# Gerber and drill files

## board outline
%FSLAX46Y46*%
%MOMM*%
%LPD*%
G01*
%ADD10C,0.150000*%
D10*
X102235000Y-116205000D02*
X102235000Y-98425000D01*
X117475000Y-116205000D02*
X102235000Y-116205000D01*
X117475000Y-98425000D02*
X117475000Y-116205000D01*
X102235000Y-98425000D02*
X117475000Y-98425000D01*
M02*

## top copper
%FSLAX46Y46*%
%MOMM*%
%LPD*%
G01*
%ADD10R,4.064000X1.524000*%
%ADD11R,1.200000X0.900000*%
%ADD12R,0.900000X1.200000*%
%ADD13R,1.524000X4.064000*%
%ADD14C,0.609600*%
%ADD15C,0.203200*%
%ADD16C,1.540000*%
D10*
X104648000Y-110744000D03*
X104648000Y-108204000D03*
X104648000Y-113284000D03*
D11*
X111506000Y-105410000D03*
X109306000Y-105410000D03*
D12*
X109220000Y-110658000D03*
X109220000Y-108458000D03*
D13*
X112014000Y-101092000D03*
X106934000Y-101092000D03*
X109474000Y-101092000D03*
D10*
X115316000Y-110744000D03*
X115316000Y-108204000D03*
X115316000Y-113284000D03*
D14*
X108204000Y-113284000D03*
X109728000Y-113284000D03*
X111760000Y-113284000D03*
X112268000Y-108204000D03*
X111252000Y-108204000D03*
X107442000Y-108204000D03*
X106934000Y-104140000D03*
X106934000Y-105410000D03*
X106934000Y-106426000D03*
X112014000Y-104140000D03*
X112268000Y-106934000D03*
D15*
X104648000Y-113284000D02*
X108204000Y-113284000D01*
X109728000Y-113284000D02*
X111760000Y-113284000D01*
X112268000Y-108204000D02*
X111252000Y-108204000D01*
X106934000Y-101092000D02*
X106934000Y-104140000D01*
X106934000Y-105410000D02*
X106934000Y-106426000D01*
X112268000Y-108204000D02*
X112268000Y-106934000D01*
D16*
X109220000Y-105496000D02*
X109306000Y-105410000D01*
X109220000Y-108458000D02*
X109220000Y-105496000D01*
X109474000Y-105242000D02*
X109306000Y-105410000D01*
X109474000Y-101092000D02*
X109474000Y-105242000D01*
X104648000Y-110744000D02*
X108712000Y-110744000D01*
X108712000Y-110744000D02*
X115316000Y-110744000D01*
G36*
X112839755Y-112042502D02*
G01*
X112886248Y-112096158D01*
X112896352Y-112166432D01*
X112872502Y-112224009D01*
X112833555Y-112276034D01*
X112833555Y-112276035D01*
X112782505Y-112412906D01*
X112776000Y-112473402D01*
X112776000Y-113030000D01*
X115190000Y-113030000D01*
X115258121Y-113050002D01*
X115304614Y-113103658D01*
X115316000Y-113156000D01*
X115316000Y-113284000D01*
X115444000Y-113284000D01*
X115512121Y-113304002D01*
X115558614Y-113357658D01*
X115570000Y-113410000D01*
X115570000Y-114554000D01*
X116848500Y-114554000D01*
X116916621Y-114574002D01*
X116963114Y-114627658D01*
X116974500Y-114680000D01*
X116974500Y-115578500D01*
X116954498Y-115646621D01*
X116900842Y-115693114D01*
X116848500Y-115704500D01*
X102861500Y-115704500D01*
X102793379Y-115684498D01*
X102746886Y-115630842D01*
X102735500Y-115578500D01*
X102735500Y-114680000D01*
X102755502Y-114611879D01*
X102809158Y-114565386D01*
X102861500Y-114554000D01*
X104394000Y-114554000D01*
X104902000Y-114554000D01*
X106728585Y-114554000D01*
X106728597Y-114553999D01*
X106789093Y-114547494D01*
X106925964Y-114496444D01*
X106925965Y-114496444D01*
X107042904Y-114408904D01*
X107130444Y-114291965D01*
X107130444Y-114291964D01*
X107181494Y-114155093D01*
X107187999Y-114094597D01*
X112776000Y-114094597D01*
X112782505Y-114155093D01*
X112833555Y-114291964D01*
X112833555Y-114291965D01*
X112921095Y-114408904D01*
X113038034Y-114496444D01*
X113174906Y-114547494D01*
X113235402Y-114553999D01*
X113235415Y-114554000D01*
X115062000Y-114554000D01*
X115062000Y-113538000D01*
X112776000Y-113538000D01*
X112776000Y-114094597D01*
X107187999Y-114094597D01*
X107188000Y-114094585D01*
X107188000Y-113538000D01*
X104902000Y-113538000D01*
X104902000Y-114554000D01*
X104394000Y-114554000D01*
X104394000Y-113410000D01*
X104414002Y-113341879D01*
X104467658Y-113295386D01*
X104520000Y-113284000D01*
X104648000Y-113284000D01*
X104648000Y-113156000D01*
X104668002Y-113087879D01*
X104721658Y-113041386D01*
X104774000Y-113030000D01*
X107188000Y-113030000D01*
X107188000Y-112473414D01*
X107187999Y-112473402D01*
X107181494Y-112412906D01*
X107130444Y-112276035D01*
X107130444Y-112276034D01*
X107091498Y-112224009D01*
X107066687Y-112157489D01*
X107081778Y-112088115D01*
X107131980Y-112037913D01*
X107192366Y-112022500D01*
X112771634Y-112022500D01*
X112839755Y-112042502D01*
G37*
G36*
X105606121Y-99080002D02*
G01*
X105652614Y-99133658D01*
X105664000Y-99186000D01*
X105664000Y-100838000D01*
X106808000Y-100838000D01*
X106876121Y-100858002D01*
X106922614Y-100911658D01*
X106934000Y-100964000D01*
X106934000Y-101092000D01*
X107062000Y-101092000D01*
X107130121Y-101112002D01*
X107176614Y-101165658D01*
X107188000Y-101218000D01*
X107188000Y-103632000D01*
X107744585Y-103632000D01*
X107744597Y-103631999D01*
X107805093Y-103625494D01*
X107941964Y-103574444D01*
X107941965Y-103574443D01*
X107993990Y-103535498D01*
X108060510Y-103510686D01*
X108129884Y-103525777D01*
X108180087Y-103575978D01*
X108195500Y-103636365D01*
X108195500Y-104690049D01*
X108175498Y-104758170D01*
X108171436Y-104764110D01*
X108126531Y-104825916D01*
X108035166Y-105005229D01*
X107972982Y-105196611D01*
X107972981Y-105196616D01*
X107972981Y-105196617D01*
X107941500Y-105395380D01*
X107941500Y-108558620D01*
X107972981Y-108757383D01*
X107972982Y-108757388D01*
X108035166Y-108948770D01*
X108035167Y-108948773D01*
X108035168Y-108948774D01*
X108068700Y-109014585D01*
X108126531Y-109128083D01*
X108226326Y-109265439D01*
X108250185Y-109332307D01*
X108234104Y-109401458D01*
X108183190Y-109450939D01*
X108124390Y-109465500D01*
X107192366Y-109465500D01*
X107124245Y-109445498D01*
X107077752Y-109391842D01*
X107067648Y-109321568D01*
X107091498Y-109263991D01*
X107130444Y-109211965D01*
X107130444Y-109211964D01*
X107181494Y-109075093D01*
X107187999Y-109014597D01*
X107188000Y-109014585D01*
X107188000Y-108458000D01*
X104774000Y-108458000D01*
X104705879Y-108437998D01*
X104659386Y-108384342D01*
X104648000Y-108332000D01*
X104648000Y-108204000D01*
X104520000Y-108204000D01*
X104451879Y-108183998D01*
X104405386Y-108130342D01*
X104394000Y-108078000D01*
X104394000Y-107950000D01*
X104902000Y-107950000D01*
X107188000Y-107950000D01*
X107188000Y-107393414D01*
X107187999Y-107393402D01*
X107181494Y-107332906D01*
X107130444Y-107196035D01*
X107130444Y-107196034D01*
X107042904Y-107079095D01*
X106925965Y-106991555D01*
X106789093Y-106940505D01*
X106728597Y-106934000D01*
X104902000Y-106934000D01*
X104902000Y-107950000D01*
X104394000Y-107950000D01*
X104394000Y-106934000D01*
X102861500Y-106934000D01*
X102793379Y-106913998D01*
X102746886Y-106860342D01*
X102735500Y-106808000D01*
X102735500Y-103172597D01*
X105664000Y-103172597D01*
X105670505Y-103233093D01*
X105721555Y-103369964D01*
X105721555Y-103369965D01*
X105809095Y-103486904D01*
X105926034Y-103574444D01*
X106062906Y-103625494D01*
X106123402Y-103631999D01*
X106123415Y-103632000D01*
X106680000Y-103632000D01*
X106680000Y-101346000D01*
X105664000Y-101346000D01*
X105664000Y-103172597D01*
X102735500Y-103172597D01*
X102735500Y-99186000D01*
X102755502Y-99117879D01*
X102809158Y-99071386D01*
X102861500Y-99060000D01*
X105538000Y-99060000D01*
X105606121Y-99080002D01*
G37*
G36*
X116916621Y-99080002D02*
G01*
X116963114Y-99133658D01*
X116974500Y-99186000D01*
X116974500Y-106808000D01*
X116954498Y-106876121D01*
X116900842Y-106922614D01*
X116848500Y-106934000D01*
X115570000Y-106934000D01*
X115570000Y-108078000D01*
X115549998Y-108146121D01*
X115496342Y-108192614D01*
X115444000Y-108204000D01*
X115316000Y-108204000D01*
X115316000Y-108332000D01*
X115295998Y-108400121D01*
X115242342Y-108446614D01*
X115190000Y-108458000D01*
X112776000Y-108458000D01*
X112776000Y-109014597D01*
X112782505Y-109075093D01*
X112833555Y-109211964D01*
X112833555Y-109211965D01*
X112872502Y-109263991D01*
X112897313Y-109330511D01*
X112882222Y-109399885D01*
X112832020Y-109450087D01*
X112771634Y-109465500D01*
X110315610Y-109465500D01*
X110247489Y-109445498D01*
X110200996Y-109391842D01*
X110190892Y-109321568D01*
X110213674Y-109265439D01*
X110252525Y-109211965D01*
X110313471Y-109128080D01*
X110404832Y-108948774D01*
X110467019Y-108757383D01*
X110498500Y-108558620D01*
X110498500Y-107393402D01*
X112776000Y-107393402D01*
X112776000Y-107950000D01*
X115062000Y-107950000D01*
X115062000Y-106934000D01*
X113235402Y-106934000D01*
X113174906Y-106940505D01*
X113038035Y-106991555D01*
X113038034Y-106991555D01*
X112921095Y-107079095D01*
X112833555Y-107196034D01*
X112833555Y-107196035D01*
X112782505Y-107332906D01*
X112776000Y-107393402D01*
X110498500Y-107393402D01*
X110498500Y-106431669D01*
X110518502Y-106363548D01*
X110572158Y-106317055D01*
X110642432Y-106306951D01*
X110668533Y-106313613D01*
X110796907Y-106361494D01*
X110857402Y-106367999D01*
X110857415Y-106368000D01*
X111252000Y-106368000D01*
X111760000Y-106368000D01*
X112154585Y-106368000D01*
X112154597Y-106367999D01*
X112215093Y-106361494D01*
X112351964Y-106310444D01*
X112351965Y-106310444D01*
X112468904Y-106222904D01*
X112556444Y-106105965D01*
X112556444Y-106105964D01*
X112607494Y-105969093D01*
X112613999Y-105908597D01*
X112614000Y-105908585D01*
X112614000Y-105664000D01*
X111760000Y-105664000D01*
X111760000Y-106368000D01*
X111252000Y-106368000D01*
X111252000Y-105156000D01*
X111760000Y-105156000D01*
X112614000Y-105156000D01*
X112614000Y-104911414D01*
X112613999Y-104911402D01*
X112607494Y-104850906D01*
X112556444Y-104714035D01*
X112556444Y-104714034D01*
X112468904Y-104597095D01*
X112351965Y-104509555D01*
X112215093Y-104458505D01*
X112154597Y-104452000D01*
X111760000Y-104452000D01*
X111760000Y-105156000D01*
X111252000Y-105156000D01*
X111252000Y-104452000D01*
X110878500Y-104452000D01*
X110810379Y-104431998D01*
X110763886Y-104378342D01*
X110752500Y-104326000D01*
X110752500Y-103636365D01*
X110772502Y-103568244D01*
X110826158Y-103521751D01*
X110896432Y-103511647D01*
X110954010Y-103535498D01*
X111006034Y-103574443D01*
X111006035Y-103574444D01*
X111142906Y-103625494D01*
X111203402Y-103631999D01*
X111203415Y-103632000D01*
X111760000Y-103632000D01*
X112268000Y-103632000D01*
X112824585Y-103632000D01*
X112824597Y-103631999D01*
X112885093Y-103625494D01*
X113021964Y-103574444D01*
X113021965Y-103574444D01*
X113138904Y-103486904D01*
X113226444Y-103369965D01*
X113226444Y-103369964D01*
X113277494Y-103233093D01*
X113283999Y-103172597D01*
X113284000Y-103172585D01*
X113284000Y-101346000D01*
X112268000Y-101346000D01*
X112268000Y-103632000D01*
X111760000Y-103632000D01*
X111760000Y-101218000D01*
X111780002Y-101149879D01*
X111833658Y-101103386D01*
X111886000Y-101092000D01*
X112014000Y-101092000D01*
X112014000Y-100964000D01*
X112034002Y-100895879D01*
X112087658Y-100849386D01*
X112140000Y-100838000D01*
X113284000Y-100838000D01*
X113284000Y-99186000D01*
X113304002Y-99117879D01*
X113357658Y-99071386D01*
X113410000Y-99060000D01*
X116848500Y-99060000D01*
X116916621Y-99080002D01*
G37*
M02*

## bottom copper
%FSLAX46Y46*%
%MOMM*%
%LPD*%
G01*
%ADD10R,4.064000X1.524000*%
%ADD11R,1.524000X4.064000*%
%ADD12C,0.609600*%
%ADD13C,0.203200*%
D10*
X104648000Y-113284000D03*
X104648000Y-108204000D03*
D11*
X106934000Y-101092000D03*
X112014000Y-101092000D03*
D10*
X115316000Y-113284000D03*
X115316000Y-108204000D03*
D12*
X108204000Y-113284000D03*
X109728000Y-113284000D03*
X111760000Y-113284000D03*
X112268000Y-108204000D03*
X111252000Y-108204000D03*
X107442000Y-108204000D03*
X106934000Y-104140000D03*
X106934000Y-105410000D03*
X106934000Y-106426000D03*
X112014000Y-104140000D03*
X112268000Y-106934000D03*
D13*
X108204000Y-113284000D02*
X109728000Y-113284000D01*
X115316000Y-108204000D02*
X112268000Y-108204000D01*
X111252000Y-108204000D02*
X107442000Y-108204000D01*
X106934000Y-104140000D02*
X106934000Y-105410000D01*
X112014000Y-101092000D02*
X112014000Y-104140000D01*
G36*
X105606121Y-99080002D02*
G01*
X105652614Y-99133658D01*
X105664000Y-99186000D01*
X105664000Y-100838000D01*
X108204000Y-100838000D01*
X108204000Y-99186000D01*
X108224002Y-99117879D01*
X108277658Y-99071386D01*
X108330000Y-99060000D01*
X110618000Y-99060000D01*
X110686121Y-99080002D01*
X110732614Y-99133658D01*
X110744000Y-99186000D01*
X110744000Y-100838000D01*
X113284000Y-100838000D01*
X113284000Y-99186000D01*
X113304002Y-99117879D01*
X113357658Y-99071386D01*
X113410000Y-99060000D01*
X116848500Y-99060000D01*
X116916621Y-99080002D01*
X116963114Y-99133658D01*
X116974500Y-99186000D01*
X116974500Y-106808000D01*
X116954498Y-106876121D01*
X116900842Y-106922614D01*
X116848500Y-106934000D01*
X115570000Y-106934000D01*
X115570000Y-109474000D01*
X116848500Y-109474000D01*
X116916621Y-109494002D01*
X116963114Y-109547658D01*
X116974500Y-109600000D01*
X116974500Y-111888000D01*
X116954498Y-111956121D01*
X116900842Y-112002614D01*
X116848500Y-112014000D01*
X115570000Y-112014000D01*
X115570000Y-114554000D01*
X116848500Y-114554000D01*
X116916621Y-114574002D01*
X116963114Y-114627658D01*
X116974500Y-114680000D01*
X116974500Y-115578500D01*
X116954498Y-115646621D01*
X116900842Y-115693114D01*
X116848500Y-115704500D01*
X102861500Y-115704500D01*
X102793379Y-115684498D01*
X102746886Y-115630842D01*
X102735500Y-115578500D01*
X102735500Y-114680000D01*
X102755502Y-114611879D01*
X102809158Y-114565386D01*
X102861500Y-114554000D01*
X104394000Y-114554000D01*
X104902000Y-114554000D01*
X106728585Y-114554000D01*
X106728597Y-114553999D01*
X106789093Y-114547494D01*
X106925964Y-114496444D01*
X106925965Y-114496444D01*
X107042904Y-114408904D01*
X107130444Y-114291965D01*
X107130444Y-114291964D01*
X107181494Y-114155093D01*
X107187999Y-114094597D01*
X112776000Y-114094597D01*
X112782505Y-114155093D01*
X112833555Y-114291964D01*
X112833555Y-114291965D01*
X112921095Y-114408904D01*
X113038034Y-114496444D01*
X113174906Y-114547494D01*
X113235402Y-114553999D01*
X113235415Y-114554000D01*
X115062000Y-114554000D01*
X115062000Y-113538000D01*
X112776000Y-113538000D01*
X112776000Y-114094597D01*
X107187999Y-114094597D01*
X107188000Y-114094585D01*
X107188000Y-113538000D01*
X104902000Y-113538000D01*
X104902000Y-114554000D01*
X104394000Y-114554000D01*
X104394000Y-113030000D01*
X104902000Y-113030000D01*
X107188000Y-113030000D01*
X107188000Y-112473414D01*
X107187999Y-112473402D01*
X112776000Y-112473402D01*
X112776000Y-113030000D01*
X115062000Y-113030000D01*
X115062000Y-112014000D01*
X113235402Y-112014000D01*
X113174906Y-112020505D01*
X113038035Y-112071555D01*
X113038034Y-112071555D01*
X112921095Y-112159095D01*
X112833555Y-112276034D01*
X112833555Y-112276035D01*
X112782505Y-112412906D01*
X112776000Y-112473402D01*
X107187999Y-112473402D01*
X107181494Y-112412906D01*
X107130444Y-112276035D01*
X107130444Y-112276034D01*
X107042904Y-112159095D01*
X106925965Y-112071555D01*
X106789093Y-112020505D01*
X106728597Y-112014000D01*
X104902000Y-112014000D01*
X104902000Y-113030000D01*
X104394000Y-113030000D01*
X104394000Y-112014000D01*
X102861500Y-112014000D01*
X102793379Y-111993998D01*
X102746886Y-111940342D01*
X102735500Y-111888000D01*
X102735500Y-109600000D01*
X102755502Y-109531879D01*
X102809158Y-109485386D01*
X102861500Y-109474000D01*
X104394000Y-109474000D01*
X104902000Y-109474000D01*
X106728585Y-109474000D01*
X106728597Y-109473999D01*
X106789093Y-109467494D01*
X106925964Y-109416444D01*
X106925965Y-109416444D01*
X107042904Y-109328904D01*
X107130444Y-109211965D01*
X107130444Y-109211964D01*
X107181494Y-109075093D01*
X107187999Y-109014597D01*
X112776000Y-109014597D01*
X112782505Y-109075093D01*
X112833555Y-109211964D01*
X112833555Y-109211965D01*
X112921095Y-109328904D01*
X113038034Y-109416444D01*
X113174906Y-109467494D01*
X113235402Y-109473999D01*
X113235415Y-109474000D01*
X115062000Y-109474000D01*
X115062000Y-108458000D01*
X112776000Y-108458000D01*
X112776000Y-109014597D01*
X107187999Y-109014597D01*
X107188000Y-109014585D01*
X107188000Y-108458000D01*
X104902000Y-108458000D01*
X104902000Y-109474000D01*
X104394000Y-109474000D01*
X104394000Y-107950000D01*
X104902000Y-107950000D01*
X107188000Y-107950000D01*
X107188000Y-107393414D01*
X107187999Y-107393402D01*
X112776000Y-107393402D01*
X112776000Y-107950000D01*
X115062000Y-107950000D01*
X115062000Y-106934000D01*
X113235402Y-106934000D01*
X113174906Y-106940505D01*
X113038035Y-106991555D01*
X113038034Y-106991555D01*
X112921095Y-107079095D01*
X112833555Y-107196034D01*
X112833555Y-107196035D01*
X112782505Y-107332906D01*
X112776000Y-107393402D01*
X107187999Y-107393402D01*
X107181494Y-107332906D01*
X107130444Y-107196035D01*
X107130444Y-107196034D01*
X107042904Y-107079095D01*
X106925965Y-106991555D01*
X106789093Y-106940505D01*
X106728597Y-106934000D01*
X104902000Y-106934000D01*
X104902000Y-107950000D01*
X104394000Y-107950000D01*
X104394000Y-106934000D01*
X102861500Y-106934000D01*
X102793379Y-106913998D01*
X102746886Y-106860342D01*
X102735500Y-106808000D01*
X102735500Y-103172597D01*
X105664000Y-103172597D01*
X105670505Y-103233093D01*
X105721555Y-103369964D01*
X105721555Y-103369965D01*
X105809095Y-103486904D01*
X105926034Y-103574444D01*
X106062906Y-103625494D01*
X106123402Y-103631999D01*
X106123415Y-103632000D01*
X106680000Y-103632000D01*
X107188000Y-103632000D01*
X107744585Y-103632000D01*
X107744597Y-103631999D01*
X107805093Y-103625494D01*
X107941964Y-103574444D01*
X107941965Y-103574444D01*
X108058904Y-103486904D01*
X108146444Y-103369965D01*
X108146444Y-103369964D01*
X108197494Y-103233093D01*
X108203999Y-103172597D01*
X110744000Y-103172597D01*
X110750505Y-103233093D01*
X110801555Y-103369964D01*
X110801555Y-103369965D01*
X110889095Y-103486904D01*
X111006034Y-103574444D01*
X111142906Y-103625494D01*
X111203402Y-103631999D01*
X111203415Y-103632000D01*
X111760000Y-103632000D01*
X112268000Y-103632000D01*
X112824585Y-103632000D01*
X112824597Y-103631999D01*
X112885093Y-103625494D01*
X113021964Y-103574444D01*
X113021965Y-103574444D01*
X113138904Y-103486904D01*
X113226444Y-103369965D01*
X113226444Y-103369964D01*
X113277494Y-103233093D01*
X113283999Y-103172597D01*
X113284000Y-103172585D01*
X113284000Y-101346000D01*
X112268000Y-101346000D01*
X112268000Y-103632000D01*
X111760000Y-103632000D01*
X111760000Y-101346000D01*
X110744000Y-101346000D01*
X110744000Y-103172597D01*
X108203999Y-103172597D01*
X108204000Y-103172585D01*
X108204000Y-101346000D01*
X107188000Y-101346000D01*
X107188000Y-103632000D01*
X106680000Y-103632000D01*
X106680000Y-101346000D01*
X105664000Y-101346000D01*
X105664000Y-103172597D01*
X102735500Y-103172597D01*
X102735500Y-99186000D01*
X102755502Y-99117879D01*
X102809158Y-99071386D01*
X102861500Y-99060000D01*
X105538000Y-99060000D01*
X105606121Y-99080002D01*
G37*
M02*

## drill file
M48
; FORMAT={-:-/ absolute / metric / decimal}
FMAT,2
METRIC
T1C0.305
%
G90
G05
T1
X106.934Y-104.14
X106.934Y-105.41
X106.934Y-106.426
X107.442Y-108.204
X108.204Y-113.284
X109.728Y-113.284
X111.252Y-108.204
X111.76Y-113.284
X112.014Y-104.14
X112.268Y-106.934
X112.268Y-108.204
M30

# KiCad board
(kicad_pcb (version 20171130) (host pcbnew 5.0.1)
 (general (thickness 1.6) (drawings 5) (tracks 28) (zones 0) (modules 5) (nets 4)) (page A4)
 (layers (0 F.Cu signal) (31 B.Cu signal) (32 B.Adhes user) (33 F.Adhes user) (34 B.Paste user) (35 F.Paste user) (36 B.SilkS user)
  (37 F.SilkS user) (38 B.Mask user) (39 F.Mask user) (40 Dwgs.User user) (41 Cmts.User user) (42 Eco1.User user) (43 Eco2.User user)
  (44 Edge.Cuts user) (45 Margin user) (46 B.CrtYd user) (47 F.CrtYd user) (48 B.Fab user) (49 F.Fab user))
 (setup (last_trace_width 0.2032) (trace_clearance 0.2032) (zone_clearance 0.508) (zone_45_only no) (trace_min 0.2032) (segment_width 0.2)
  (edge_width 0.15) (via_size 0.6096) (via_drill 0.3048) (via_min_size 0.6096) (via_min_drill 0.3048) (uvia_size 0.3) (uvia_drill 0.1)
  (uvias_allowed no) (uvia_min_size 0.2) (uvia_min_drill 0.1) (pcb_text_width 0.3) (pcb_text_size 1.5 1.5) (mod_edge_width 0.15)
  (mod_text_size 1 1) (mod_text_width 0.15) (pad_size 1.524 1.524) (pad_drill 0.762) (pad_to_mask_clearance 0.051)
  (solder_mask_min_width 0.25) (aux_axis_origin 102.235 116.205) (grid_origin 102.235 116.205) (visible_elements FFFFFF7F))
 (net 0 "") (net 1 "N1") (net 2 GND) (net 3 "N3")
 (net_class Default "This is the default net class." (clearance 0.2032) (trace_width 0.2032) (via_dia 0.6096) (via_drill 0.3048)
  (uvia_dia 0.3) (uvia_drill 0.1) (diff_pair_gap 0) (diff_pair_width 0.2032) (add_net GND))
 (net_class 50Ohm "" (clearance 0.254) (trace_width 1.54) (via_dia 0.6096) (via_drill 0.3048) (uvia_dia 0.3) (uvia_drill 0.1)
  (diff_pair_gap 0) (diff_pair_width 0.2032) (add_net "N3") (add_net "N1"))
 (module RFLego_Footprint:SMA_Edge (layer F.Cu) (at 102.616 110.744)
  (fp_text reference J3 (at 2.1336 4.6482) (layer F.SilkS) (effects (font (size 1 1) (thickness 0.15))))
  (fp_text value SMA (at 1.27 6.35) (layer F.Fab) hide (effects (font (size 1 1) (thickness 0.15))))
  (pad 1 smd rect (at 2.032 0) (size 4.064 1.524) (layers F.Cu F.Mask) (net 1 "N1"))
  (pad 2 smd rect (at 2.032 -2.54) (size 4.064 1.524) (layers F.Cu F.Mask) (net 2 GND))
  (pad 2 smd rect (at 2.032 2.54) (size 4.064 1.524) (layers B.Cu B.Mask) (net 2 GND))
  (pad 2 smd rect (at 2.032 -2.54) (size 4.064 1.524) (layers B.Cu B.Mask) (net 2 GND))
  (pad 2 smd rect (at 2.032 2.54) (size 4.064 1.524) (layers F.Cu F.Mask) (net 2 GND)))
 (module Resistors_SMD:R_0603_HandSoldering (layer F.Cu) (at 110.406 105.41 180)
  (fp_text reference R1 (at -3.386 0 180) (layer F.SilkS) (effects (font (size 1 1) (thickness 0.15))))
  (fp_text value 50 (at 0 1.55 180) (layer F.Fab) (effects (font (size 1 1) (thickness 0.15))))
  (pad 1 smd rect (at -1.1 0 180) (size 1.2 0.9) (layers F.Cu F.Paste F.Mask) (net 2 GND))
  (pad 2 smd rect (at 1.1 0 180) (size 1.2 0.9) (layers F.Cu F.Paste F.Mask) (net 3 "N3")))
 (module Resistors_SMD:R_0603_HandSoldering (layer F.Cu) (at 109.22 109.558 270)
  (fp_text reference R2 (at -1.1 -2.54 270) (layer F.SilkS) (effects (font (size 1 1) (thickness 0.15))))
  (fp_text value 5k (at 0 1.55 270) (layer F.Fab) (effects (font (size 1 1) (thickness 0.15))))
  (pad 2 smd rect (at 1.1 0 270) (size 1.2 0.9) (layers F.Cu F.Paste F.Mask) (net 1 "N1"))
  (pad 1 smd rect (at -1.1 0 270) (size 1.2 0.9) (layers F.Cu F.Paste F.Mask) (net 3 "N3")))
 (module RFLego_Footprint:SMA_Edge (layer F.Cu) (at 109.474 103.124 90)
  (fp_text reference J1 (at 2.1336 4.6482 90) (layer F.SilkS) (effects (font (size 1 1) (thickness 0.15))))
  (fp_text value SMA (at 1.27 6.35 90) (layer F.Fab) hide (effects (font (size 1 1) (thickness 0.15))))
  (pad 2 smd rect (at 2.032 2.54 90) (size 4.064 1.524) (layers F.Cu F.Mask) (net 2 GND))
  (pad 2 smd rect (at 2.032 -2.54 90) (size 4.064 1.524) (layers B.Cu B.Mask) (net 2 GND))
  (pad 2 smd rect (at 2.032 2.54 90) (size 4.064 1.524) (layers B.Cu B.Mask) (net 2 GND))
  (pad 2 smd rect (at 2.032 -2.54 90) (size 4.064 1.524) (layers F.Cu F.Mask) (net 2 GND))
  (pad 1 smd rect (at 2.032 0 90) (size 4.064 1.524) (layers F.Cu F.Mask) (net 3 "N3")))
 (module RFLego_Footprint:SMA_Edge (layer F.Cu) (at 113.284 110.744)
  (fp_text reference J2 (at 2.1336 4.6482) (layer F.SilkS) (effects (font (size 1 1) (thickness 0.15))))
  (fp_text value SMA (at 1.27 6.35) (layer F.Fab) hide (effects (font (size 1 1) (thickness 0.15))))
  (pad 1 smd rect (at 2.032 0) (size 4.064 1.524) (layers F.Cu F.Mask) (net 1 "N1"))
  (pad 2 smd rect (at 2.032 -2.54) (size 4.064 1.524) (layers F.Cu F.Mask) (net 2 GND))
  (pad 2 smd rect (at 2.032 2.54) (size 4.064 1.524) (layers B.Cu B.Mask) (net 2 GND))
  (pad 2 smd rect (at 2.032 -2.54) (size 4.064 1.524) (layers B.Cu B.Mask) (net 2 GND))
  (pad 2 smd rect (at 2.032 2.54) (size 4.064 1.524) (layers F.Cu F.Mask) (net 2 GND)))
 (gr_line (start 102.235 116.205) (end 102.235 98.425) (layer Edge.Cuts) (width 0.15))
 (gr_line (start 117.475 116.205) (end 102.235 116.205) (layer Edge.Cuts) (width 0.15))
 (gr_line (start 117.475 98.425) (end 117.475 116.205) (layer Edge.Cuts) (width 0.15))
 (gr_line (start 102.235 98.425) (end 117.475 98.425) (layer Edge.Cuts) (width 0.15))
 (via (at 108.204 113.284) (size 0.6096) (drill 0.3048) (layers F.Cu B.Cu) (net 2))
 (segment (start 104.648 113.284) (end 108.204 113.284) (width 0.2032) (layer F.Cu) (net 2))
 (via (at 109.728 113.284) (size 0.6096) (drill 0.3048) (layers F.Cu B.Cu) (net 2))
 (segment (start 108.204 113.284) (end 109.728 113.284) (width 0.2032) (layer B.Cu) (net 2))
 (via (at 111.76 113.284) (size 0.6096) (drill 0.3048) (layers F.Cu B.Cu) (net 2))
 (segment (start 109.728 113.284) (end 111.76 113.284) (width 0.2032) (layer F.Cu) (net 2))
 (via (at 112.268 108.204) (size 0.6096) (drill 0.3048) (layers F.Cu B.Cu) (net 2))
 (segment (start 115.316 108.204) (end 112.268 108.204) (width 0.2032) (layer B.Cu) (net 2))
 (via (at 111.252 108.204) (size 0.6096) (drill 0.3048) (layers F.Cu B.Cu) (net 2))
 (segment (start 112.268 108.204) (end 111.252 108.204) (width 0.2032) (layer F.Cu) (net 2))
 (via (at 107.442 108.204) (size 0.6096) (drill 0.3048) (layers F.Cu B.Cu) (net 2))
 (segment (start 111.252 108.204) (end 107.442 108.204) (width 0.2032) (layer B.Cu) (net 2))
 (via (at 106.934 104.14) (size 0.6096) (drill 0.3048) (layers F.Cu B.Cu) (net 2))
 (segment (start 106.934 101.092) (end 106.934 104.14) (width 0.2032) (layer F.Cu) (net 2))
 (via (at 106.934 105.41) (size 0.6096) (drill 0.3048) (layers F.Cu B.Cu) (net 2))
 (segment (start 106.934 104.14) (end 106.934 105.41) (width 0.2032) (layer B.Cu) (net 2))
 (via (at 106.934 106.426) (size 0.6096) (drill 0.3048) (layers F.Cu B.Cu) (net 2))
 (segment (start 106.934 105.41) (end 106.934 106.426) (width 0.2032) (layer F.Cu) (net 2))
 (via (at 112.014 104.14) (size 0.6096) (drill 0.3048) (layers F.Cu B.Cu) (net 2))
 (segment (start 112.014 101.092) (end 112.014 104.14) (width 0.2032) (layer B.Cu) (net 2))
 (via (at 112.268 106.934) (size 0.6096) (drill 0.3048) (layers F.Cu B.Cu) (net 2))
 (segment (start 112.268 108.204) (end 112.268 106.934) (width 0.2032) (layer F.Cu) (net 2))
 (segment (start 109.22 105.496) (end 109.306 105.41) (width 1.54) (layer F.Cu) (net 3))
 (segment (start 109.22 108.458) (end 109.22 105.496) (width 1.54) (layer F.Cu) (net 3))
 (segment (start 109.474 105.242) (end 109.306 105.41) (width 1.54) (layer F.Cu) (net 3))
 (segment (start 109.474 101.092) (end 109.474 105.242) (width 1.54) (layer F.Cu) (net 3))
 (segment (start 104.648 110.744) (end 108.712 110.744) (width 1.54) (layer F.Cu) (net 1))
 (segment (start 108.712 110.744) (end 115.316 110.744) (width 1.54) (layer F.Cu) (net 1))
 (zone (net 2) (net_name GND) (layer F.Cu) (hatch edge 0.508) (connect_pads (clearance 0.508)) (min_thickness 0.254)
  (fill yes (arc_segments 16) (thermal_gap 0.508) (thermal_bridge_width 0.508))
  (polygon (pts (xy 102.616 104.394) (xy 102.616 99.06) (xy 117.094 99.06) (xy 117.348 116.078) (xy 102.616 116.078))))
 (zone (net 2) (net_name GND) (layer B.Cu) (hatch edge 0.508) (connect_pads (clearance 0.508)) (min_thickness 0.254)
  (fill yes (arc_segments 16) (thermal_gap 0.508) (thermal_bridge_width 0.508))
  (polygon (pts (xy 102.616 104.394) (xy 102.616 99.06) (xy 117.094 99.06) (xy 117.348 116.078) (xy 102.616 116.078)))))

